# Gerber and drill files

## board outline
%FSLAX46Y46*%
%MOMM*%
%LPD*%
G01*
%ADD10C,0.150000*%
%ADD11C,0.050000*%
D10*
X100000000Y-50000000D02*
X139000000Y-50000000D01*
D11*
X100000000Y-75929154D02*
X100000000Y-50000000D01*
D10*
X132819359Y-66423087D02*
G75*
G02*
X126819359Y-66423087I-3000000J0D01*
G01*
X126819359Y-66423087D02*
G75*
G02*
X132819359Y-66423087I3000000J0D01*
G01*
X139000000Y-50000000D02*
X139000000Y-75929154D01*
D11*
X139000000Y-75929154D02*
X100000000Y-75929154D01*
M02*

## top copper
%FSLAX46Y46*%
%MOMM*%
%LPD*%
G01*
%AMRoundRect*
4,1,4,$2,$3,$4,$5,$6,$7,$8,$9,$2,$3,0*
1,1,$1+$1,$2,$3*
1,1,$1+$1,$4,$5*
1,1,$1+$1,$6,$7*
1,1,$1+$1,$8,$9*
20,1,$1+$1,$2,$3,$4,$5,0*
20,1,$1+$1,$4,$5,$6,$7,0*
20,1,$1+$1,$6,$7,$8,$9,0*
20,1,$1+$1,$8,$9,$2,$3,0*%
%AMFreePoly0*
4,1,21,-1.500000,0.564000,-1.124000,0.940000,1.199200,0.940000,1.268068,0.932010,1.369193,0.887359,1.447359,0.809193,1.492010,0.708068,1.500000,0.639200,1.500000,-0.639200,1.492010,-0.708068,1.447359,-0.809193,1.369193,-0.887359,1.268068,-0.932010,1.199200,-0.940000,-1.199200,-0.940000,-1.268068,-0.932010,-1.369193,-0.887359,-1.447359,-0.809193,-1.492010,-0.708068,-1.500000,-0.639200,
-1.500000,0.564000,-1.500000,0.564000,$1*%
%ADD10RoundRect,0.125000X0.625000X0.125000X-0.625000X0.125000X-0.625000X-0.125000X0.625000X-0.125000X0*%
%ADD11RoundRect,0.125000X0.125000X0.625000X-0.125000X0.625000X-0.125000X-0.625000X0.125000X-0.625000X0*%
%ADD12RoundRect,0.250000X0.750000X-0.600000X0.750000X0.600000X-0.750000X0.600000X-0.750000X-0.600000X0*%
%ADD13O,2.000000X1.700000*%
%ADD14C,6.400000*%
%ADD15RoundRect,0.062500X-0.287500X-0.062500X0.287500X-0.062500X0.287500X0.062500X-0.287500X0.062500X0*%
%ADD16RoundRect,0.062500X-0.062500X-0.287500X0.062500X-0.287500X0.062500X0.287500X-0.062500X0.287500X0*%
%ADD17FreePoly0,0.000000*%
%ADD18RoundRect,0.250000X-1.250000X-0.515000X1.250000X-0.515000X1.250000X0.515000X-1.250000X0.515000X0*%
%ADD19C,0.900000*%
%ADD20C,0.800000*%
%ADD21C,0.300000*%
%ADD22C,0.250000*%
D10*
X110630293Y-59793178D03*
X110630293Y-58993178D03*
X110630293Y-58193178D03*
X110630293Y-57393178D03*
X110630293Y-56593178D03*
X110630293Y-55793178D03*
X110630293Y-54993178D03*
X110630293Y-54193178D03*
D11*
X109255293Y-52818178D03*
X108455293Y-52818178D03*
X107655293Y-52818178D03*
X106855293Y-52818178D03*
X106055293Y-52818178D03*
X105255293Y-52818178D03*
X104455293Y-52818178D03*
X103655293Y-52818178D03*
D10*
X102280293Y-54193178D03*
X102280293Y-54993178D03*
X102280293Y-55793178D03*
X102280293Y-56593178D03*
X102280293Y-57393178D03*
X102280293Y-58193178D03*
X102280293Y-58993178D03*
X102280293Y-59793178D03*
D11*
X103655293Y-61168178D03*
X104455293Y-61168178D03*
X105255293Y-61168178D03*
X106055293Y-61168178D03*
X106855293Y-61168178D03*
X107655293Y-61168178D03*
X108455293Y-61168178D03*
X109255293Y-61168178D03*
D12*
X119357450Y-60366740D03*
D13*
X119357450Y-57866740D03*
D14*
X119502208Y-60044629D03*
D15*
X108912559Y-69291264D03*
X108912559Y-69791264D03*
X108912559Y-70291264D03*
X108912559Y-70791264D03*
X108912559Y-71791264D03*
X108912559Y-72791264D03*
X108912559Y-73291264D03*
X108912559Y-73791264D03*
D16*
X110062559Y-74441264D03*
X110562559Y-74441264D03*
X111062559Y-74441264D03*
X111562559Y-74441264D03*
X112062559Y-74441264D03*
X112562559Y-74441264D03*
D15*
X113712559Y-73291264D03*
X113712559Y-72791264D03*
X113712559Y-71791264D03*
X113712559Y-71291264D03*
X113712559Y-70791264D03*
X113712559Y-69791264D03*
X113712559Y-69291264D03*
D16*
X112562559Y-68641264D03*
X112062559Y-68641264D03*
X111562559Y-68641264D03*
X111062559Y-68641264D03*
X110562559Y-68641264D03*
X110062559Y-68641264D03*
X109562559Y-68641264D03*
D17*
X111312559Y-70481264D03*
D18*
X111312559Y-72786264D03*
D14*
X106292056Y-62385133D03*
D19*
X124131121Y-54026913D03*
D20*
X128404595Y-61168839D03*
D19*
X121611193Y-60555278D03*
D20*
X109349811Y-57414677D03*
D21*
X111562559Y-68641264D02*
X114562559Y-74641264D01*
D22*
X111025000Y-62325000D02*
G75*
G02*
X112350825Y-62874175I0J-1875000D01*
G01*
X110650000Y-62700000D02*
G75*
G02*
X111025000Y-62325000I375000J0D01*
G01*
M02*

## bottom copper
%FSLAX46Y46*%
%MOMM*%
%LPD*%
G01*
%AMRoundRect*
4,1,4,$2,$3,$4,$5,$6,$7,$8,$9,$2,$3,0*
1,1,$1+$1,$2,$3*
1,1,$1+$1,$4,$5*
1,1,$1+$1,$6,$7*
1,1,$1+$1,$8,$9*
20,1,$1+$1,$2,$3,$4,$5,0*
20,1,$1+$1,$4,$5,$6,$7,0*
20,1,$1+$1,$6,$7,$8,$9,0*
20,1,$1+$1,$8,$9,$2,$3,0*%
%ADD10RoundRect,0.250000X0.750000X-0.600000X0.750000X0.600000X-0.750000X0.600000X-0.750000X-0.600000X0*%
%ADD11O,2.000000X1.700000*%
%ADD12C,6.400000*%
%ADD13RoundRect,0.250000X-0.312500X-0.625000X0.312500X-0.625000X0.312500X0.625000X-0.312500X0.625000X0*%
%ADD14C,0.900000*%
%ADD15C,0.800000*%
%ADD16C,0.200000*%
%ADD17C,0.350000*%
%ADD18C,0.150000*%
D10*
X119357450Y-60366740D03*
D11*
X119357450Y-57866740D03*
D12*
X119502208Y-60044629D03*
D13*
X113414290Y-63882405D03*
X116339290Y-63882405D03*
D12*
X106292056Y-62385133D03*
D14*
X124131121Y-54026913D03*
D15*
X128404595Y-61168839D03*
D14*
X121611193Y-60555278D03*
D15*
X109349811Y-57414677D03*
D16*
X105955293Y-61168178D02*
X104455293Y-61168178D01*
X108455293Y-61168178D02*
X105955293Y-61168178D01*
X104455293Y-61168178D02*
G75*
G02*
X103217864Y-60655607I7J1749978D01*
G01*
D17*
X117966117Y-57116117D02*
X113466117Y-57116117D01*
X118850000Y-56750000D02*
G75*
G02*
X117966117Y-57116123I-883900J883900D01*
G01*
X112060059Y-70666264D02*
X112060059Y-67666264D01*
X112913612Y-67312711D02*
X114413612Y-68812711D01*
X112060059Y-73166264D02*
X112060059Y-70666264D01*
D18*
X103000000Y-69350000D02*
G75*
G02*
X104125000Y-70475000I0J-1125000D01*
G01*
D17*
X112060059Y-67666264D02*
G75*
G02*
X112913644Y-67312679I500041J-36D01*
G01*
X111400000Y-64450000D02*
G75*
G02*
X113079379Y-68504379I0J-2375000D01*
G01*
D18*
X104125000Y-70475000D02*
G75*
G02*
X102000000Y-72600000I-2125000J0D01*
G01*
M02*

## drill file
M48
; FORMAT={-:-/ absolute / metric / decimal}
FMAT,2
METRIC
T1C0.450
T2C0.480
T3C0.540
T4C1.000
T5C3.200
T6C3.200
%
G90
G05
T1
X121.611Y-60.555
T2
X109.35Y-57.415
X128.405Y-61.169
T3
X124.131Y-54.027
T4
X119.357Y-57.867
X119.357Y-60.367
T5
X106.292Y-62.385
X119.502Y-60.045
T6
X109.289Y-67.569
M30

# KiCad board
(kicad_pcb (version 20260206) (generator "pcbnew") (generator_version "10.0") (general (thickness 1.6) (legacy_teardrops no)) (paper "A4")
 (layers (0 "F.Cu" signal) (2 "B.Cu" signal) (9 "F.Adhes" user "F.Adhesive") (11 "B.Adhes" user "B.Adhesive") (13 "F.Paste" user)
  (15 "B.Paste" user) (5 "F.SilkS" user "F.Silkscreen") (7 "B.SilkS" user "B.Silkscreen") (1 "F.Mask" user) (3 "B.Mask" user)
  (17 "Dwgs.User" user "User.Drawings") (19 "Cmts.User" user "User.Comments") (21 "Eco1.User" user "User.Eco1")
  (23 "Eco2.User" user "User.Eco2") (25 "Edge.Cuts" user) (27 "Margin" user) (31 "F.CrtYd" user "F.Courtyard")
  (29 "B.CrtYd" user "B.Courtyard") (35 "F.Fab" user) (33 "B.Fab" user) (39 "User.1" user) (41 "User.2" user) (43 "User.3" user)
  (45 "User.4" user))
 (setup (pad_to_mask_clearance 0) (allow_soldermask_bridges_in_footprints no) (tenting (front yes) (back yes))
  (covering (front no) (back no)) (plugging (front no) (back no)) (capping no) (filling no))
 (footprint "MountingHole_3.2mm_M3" (layer "F.Cu") (at 109.289246 67.568769)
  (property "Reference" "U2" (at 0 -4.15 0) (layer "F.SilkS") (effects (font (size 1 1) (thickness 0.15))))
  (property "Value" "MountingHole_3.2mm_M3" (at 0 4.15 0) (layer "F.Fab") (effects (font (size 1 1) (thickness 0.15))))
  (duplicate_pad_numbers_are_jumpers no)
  (pad "" np_thru_hole circle (at 0 0) (size 3.2 3.2) (drill 3.2) (layers "*.Cu" "*.Mask")))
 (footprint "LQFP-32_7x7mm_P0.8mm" (layer "F.Cu") (at 106.455293 56.993178 180)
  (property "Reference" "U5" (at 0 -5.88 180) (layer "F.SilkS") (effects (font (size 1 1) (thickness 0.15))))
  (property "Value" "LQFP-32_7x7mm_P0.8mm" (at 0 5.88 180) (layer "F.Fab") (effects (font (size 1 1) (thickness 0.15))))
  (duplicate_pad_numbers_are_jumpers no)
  (pad "1" smd roundrect (at -4.175 -2.8 180) (size 1.5 0.5) (layers "F.Cu" "F.Mask" "F.Paste") (roundrect_rratio 0.25) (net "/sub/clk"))
  (pad "2" smd roundrect (at -4.175 -2 180) (size 1.5 0.5) (layers "F.Cu" "F.Mask" "F.Paste") (roundrect_rratio 0.25) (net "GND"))
  (pad "3" smd roundrect (at -4.175 -1.2 180) (size 1.5 0.5) (layers "F.Cu" "F.Mask" "F.Paste") (roundrect_rratio 0.25) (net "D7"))
  (pad "4" smd roundrect (at -4.175 -0.4 180) (size 1.5 0.5) (layers "F.Cu" "F.Mask" "F.Paste") (roundrect_rratio 0.25) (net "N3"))
  (pad "5" smd roundrect (at -4.175 0.4 180) (size 1.5 0.5) (layers "F.Cu" "F.Mask" "F.Paste") (roundrect_rratio 0.25))
  (pad "6" smd roundrect (at -4.175 1.2 180) (size 1.5 0.5) (layers "F.Cu" "F.Mask" "F.Paste") (roundrect_rratio 0.25) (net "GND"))
  (pad "7" smd roundrect (at -4.175 2 180) (size 1.5 0.5) (layers "F.Cu" "F.Mask" "F.Paste") (roundrect_rratio 0.25))
  (pad "8" smd roundrect (at -4.175 2.8 180) (size 1.5 0.5) (layers "F.Cu" "F.Mask" "F.Paste") (roundrect_rratio 0.25) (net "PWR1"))
  (pad "9" smd roundrect (at -2.8 4.175 180) (size 0.5 1.5) (layers "F.Cu" "F.Mask" "F.Paste") (roundrect_rratio 0.25) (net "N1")
   (clearance 0.35))
  (pad "10" smd roundrect (at -2 4.175 180) (size 0.5 1.5) (layers "F.Cu" "F.Mask" "F.Paste") (roundrect_rratio 0.25) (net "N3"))
  (pad "11" smd roundrect (at -1.2 4.175 180) (size 0.5 1.5) (layers "F.Cu" "F.Mask" "F.Paste") (roundrect_rratio 0.25) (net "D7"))
  (pad "12" smd roundrect (at -0.4 4.175 180) (size 0.5 1.5) (layers "F.Cu" "F.Mask" "F.Paste") (roundrect_rratio 0.25) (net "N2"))
  (pad "13" smd roundrect (at 0.4 4.175 180) (size 0.5 1.5) (layers "F.Cu" "F.Mask" "F.Paste") (roundrect_rratio 0.25) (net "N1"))
  (pad "14" smd roundrect (at 1.2 4.175 180) (size 0.5 1.5) (layers "F.Cu" "F.Mask" "F.Paste") (roundrect_rratio 0.25) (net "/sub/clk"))
  (pad "15" smd roundrect (at 2 4.175 180) (size 0.5 1.5) (layers "F.Cu" "F.Mask" "F.Paste") (roundrect_rratio 0.25))
  (pad "16" smd roundrect (at 2.8 4.175 180) (size 0.5 1.5) (layers "F.Cu" "F.Mask" "F.Paste") (roundrect_rratio 0.25))
  (pad "17" smd roundrect (at 4.175 2.8 180) (size 1.5 0.5) (layers "F.Cu" "F.Mask" "F.Paste") (roundrect_rratio 0.25) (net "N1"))
  (pad "18" smd roundrect (at 4.175 2 180) (size 1.5 0.5) (layers "F.Cu" "F.Mask" "F.Paste") (roundrect_rratio 0.25) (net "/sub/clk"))
  (pad "19" smd roundrect (at 4.175 1.2 180) (size 1.5 0.5) (layers "F.Cu" "F.Mask" "F.Paste") (roundrect_rratio 0.25) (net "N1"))
  (pad "20" smd roundrect (at 4.175 0.4 180) (size 1.5 0.5) (layers "F.Cu" "F.Mask" "F.Paste") (roundrect_rratio 0.25) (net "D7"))
  (pad "21" smd roundrect (at 4.175 -0.4 180) (size 1.5 0.5) (layers "F.Cu" "F.Mask" "F.Paste") (roundrect_rratio 0.25) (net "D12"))
  (pad "22" smd roundrect (at 4.175 -1.2 180) (size 1.5 0.5) (layers "F.Cu" "F.Mask" "F.Paste") (roundrect_rratio 0.25))
  (pad "23" smd roundrect (at 4.175 -2 180) (size 1.5 0.5) (layers "F.Cu" "F.Mask" "F.Paste") (roundrect_rratio 0.25))
  (pad "24" smd roundrect (at 4.175 -2.8 180) (size 1.5 0.5) (layers "F.Cu" "F.Mask" "F.Paste") (roundrect_rratio 0.25))
  (pad "25" smd roundrect (at 2.8 -4.175 180) (size 0.5 1.5) (layers "F.Cu" "F.Mask" "F.Paste") (roundrect_rratio 0.25) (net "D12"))
  (pad "26" smd roundrect (at 2 -4.175 180) (size 0.5 1.5) (layers "F.Cu" "F.Mask" "F.Paste") (roundrect_rratio 0.25) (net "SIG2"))
  (pad "27" smd roundrect (at 1.2 -4.175 180) (size 0.5 1.5) (layers "F.Cu" "F.Mask" "F.Paste") (roundrect_rratio 0.25) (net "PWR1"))
  (pad "28" smd roundrect (at 0.4 -4.175 180) (size 0.5 1.5) (layers "F.Cu" "F.Mask" "F.Paste") (roundrect_rratio 0.25) (clearance 0.35))
  (pad "29" smd roundrect (at -0.4 -4.175 180) (size 0.5 1.5) (layers "F.Cu" "F.Mask" "F.Paste") (roundrect_rratio 0.25) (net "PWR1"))
  (pad "30" smd roundrect (at -1.2 -4.175 180) (size 0.5 1.5) (layers "F.Cu" "F.Mask" "F.Paste") (roundrect_rratio 0.25) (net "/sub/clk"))
  (pad "31" smd roundrect (at -2 -4.175 180) (size 0.5 1.5) (layers "F.Cu" "F.Mask" "F.Paste") (roundrect_rratio 0.25) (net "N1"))
  (pad "32" smd roundrect (at -2.8 -4.175 180) (size 0.5 1.5) (layers "F.Cu" "F.Mask" "F.Paste") (roundrect_rratio 0.25) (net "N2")))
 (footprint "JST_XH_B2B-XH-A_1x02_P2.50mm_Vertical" (layer "F.Cu") (at 119.35745 60.36674 90)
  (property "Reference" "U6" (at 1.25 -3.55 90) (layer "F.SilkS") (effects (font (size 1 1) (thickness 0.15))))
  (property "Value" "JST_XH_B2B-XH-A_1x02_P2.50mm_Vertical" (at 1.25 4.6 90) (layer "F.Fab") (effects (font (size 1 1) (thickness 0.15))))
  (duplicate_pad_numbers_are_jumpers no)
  (pad "1" thru_hole roundrect (at 0 0 90) (size 1.7 2) (drill 1) (layers "*.Cu" "*.Mask") (remove_unused_layers no)
   (roundrect_rratio 0.147059) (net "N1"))
  (pad "2" thru_hole oval (at 2.5 0 90) (size 1.7 2) (drill 1) (layers "*.Cu" "*.Mask") (remove_unused_layers no)))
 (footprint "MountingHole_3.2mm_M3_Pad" (layer "F.Cu") (at 119.502208 60.044629)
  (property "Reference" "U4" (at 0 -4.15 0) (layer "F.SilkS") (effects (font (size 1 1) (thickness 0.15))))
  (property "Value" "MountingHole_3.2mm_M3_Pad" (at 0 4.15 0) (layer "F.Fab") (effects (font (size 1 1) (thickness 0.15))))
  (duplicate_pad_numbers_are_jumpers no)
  (pad "1" thru_hole circle (at 0 0) (size 6.4 6.4) (drill 3.2) (layers "*.Cu" "*.Mask") (remove_unused_layers no) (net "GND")
   (zone_connect 2)))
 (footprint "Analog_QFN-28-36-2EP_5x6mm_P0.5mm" (layer "F.Cu") (at 111.312559 71.541264)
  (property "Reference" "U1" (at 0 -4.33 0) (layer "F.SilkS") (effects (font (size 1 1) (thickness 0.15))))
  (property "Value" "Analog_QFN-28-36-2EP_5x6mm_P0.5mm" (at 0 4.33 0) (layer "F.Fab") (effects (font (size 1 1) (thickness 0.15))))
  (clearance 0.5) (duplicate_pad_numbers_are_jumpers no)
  (pad "" smd roundrect (at -0.75 -1.53) (size 1.21 0.76) (layers "F.Paste") (roundrect_rratio 0.25) (chamfer_ratio 0.4) (chamfer top_left)
   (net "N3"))
  (pad "" smd roundrect (at -0.75 -0.59) (size 1.21 0.76) (layers "F.Paste") (roundrect_rratio 0.25) (clearance 0.1))
  (pad "" smd roundrect (at -0.7475 0.875) (size 1.205 0.55) (layers "F.Paste") (roundrect_rratio 0.25) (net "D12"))
  (pad "" smd roundrect (at -0.7475 1.625) (size 1.205 0.55) (layers "F.Paste") (roundrect_rratio 0.25) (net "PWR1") (clearance 0.35))
  (pad "" smd roundrect (at 0.7475 0.875) (size 1.205 0.55) (layers "F.Paste") (roundrect_rratio 0.25) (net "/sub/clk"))
  (pad "" smd roundrect (at 0.7475 1.625) (size 1.205 0.55) (layers "F.Paste") (roundrect_rratio 0.25) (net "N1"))
  (pad "" smd roundrect (at 0.75 -1.53) (size 1.21 0.76) (layers "F.Paste") (roundrect_rratio 0.25) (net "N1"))
  (pad "" smd roundrect (at 0.75 -0.59) (size 1.21 0.76) (layers "F.Paste") (roundrect_rratio 0.25) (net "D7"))
  (pad "1" smd roundrect (at -2.4 -2.25) (size 0.7 0.25) (layers "F.Cu" "F.Mask" "F.Paste") (roundrect_rratio 0.25) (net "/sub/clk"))
  (pad "2" smd roundrect (at -2.4 -1.75) (size 0.7 0.25) (layers "F.Cu" "F.Mask" "F.Paste") (roundrect_rratio 0.25) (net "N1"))
  (pad "3" smd roundrect (at -2.4 -1.25) (size 0.7 0.25) (layers "F.Cu" "F.Mask" "F.Paste") (roundrect_rratio 0.25))
  (pad "4" smd roundrect (at -2.4 -0.75) (size 0.7 0.25) (layers "F.Cu" "F.Mask" "F.Paste") (roundrect_rratio 0.25))
  (pad "6" smd roundrect (at -2.4 0.25) (size 0.7 0.25) (layers "F.Cu" "F.Mask" "F.Paste") (roundrect_rratio 0.25) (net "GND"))
  (pad "8" smd roundrect (at -2.4 1.25) (size 0.7 0.25) (layers "F.Cu" "F.Mask" "F.Paste") (roundrect_rratio 0.25))
  (pad "9" smd roundrect (at -2.4 1.75) (size 0.7 0.25) (layers "F.Cu" "F.Mask" "F.Paste") (roundrect_rratio 0.25) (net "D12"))
  (pad "10" smd roundrect (at -2.4 2.25) (size 0.7 0.25) (layers "F.Cu" "F.Mask" "F.Paste") (roundrect_rratio 0.25) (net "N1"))
  (pad "12" smd roundrect (at -1.25 2.9) (size 0.25 0.7) (layers "F.Cu" "F.Mask" "F.Paste") (roundrect_rratio 0.25))
  (pad "13" smd roundrect (at -0.75 2.9) (size 0.25 0.7) (layers "F.Cu" "F.Mask" "F.Paste") (roundrect_rratio 0.25) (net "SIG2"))
  (pad "14" smd roundrect (at -0.25 2.9) (size 0.25 0.7) (layers "F.Cu" "F.Mask" "F.Paste") (roundrect_rratio 0.25) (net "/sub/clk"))
  (pad "15" smd roundrect (at 0.25 2.9) (size 0.25 0.7) (layers "F.Cu" "F.Mask" "F.Paste") (roundrect_rratio 0.25))
  (pad "16" smd roundrect (at 0.75 2.9) (size 0.25 0.7) (layers "F.Cu" "F.Mask" "F.Paste") (roundrect_rratio 0.25) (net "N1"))
  (pad "17" smd roundrect (at 1.25 2.9) (size 0.25 0.7) (layers "F.Cu" "F.Mask" "F.Paste") (roundrect_rratio 0.25) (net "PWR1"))
  (pad "20" smd roundrect (at 2.4 1.75) (size 0.7 0.25) (layers "F.Cu" "F.Mask" "F.Paste") (roundrect_rratio 0.25) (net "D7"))
  (pad "21" smd roundrect (at 2.4 1.25) (size 0.7 0.25) (layers "F.Cu" "F.Mask" "F.Paste") (roundrect_rratio 0.25) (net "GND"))
  (pad "23" smd roundrect (at 2.4 0.25) (size 0.7 0.25) (layers "F.Cu" "F.Mask" "F.Paste") (roundrect_rratio 0.25))
  (pad "24" smd roundrect (at 2.4 -0.25) (size 0.7 0.25) (layers "F.Cu" "F.Mask" "F.Paste") (roundrect_rratio 0.25) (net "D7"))
  (pad "25" smd roundrect (at 2.4 -0.75) (size 0.7 0.25) (layers "F.Cu" "F.Mask" "F.Paste") (roundrect_rratio 0.25) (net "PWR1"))
  (pad "27" smd roundrect (at 2.4 -1.75) (size 0.7 0.25) (layers "F.Cu" "F.Mask" "F.Paste") (roundrect_rratio 0.25) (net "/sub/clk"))
  (pad "28" smd roundrect (at 2.4 -2.25) (size 0.7 0.25) (layers "F.Cu" "F.Mask" "F.Paste") (roundrect_rratio 0.25) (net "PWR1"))
  (pad "30" smd roundrect (at 1.25 -2.9) (size 0.25 0.7) (layers "F.Cu" "F.Mask" "F.Paste") (roundrect_rratio 0.25))
  (pad "31" smd roundrect (at 0.75 -2.9) (size 0.25 0.7) (layers "F.Cu" "F.Mask" "F.Paste") (roundrect_rratio 0.25))
  (pad "32" smd roundrect (at 0.25 -2.9) (size 0.25 0.7) (layers "F.Cu" "F.Mask" "F.Paste") (roundrect_rratio 0.25))
  (pad "33" smd roundrect (at -0.25 -2.9) (size 0.25 0.7) (layers "F.Cu" "F.Mask" "F.Paste") (roundrect_rratio 0.25) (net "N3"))
  (pad "34" smd roundrect (at -0.75 -2.9) (size 0.25 0.7) (layers "F.Cu" "F.Mask" "F.Paste") (roundrect_rratio 0.25))
  (pad "35" smd roundrect (at -1.25 -2.9) (size 0.25 0.7) (layers "F.Cu" "F.Mask" "F.Paste") (roundrect_rratio 0.25))
  (pad "36" smd roundrect (at -1.75 -2.9) (size 0.25 0.7) (layers "F.Cu" "F.Mask" "F.Paste") (roundrect_rratio 0.25) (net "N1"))
  (pad "37" smd roundrect (at 0 -1.06) (size 3 1.88) (layers "F.Cu" "F.Mask") (roundrect_rratio 0.16) (chamfer_ratio 0.2) (chamfer top_left)
   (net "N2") (zone_connect 2))
  (pad "38" smd roundrect (at 0 1.245) (size 3 1.53) (layers "F.Cu" "F.Mask") (roundrect_rratio 0.1633986928) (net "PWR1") (zone_connect 2)))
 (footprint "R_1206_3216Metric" (layer "B.Cu") (at 114.87679 63.882405)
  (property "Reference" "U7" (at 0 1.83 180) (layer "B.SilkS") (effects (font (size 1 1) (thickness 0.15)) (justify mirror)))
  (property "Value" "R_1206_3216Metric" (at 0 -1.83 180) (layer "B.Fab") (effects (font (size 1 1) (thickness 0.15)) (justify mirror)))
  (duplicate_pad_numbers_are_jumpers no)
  (pad "1" smd roundrect (at -1.4625 0) (size 1.125 1.75) (layers "B.Cu" "B.Mask" "B.Paste") (roundrect_rratio 0.222222) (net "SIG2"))
  (pad "2" smd roundrect (at 1.4625 0) (size 1.125 1.75) (layers "B.Cu" "B.Mask" "B.Paste") (roundrect_rratio 0.222222) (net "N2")))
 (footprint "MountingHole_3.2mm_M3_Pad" (layer "B.Cu") (at 106.292056 62.385133 90)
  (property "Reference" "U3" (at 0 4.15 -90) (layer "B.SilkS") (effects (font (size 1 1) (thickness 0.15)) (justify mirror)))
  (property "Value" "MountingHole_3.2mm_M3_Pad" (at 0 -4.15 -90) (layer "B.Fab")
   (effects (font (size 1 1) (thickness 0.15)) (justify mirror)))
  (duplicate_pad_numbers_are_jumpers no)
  (pad "1" thru_hole circle (at 0 0 90) (size 6.4 6.4) (drill 3.2) (layers "*.Cu" "*.Mask") (remove_unused_layers no) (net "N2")
   (clearance 0.1) (zone_connect 2)))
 (gr_line (start 100 50) (end 139 50) (stroke (width 0.15) (type default)) (layer "Edge.Cuts"))
 (gr_line (start 100 75.929154) (end 100 50) (stroke (width 0.05) (type default)) (layer "Edge.Cuts"))
 (gr_circle (center 129.819359 66.423087) (end 132.819359 66.423087) (stroke (width 0.15) (type default)) (fill no) (layer "Edge.Cuts"))
 (gr_line (start 139 50) (end 139 75.929154) (stroke (width 0.15) (type default)) (layer "Edge.Cuts"))
 (gr_line (start 139 75.929154) (end 100 75.929154) (stroke (width 0.05) (type default)) (layer "Edge.Cuts"))
 (segment (start 111.562559 68.641264) (end 114.562559 74.641264) (width 0.3) (layer "F.Cu") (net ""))
 (arc (start 111.025 62.325) (mid 111.742531 62.467726) (end 112.350825 62.874175) (width 0.25) (locked yes) (layer "F.Cu") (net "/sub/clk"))
 (arc (start 110.65 62.7) (mid 110.759835 62.434835) (end 111.025 62.325) (width 0.25) (layer "F.Cu") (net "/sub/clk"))
 (segment (start 105.955293 61.168178) (end 104.455293 61.168178) (width 0.2) (layer "B.Cu") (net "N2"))
 (segment (start 108.455293 61.168178) (end 105.955293 61.168178) (width 0.2) (layer "B.Cu") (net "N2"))
 (arc (start 104.455293 61.168178) (mid 103.785597 61.034967) (end 103.217856 60.655615) (width 0.2) (layer "B.Cu") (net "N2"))
 (via (at 124.131121 54.026913) (size 0.9) (drill 0.54) (layers "F.Cu" "B.Cu") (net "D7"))
 (via (at 128.404595 61.168839) (size 0.8) (drill 0.48) (layers "F.Cu" "B.Cu") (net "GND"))
 (via (at 121.611193 60.555278) (size 0.9) (drill 0.45) (layers "F.Cu" "B.Cu") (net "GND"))
 (segment (start 117.966117 57.116117) (end 113.466117 57.116117) (width 0.35) (layer "B.Cu") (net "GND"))
 (arc (start 118.85 56.75) (mid 118.444471 57.020966) (end 117.966117 57.116117) (width 0.35) (layer "B.Cu") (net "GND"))
 (via (at 109.349811 57.414677) (size 0.8) (drill 0.48) (layers "F.Cu" "B.Cu") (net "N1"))
 (segment (start 112.060059 70.666264) (end 112.060059 67.666264) (width 0.35) (layer "B.Cu") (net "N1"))
 (segment (start 112.913612 67.312711) (end 114.413612 68.812711) (width 0.35) (layer "B.Cu") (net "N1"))
 (segment (start 112.060059 73.166264) (end 112.060059 70.666264) (width 0.35) (layer "B.Cu") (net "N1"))
 (arc (start 103 69.35) (mid 103.795495 69.679505) (end 104.125 70.475) (width 0.15) (layer "B.Cu") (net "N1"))
 (arc (start 112.060059 67.666264) (mid 112.368717 67.204324) (end 112.913612 67.312711) (width 0.35) (layer "B.Cu") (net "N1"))
 (arc (start 111.4 64.45) (mid 113.594214 65.916127) (end 113.079379 68.504379) (width 0.35) (layer "B.Cu") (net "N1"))
 (arc (start 104.125 70.475) (mid 103.502602 71.977602) (end 102 72.6) (width 0.15) (locked yes) (layer "B.Cu") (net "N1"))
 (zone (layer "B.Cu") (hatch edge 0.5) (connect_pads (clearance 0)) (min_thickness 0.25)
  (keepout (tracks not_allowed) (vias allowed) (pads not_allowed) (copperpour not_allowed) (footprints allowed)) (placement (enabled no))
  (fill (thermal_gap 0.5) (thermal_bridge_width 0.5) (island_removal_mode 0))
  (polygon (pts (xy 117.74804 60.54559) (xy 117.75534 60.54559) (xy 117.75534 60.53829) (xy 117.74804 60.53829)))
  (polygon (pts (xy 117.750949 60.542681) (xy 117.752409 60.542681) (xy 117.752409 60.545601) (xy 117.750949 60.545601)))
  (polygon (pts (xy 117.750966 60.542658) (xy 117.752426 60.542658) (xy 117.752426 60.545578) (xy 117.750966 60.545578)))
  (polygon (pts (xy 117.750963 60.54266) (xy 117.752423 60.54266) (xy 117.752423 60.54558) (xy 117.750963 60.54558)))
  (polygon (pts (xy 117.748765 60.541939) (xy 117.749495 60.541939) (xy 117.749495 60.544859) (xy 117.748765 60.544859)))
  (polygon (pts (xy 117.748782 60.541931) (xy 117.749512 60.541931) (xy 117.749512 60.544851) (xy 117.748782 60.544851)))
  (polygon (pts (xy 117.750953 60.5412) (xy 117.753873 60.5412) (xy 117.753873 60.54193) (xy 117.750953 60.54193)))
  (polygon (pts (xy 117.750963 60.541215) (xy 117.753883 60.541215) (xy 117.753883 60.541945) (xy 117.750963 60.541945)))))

